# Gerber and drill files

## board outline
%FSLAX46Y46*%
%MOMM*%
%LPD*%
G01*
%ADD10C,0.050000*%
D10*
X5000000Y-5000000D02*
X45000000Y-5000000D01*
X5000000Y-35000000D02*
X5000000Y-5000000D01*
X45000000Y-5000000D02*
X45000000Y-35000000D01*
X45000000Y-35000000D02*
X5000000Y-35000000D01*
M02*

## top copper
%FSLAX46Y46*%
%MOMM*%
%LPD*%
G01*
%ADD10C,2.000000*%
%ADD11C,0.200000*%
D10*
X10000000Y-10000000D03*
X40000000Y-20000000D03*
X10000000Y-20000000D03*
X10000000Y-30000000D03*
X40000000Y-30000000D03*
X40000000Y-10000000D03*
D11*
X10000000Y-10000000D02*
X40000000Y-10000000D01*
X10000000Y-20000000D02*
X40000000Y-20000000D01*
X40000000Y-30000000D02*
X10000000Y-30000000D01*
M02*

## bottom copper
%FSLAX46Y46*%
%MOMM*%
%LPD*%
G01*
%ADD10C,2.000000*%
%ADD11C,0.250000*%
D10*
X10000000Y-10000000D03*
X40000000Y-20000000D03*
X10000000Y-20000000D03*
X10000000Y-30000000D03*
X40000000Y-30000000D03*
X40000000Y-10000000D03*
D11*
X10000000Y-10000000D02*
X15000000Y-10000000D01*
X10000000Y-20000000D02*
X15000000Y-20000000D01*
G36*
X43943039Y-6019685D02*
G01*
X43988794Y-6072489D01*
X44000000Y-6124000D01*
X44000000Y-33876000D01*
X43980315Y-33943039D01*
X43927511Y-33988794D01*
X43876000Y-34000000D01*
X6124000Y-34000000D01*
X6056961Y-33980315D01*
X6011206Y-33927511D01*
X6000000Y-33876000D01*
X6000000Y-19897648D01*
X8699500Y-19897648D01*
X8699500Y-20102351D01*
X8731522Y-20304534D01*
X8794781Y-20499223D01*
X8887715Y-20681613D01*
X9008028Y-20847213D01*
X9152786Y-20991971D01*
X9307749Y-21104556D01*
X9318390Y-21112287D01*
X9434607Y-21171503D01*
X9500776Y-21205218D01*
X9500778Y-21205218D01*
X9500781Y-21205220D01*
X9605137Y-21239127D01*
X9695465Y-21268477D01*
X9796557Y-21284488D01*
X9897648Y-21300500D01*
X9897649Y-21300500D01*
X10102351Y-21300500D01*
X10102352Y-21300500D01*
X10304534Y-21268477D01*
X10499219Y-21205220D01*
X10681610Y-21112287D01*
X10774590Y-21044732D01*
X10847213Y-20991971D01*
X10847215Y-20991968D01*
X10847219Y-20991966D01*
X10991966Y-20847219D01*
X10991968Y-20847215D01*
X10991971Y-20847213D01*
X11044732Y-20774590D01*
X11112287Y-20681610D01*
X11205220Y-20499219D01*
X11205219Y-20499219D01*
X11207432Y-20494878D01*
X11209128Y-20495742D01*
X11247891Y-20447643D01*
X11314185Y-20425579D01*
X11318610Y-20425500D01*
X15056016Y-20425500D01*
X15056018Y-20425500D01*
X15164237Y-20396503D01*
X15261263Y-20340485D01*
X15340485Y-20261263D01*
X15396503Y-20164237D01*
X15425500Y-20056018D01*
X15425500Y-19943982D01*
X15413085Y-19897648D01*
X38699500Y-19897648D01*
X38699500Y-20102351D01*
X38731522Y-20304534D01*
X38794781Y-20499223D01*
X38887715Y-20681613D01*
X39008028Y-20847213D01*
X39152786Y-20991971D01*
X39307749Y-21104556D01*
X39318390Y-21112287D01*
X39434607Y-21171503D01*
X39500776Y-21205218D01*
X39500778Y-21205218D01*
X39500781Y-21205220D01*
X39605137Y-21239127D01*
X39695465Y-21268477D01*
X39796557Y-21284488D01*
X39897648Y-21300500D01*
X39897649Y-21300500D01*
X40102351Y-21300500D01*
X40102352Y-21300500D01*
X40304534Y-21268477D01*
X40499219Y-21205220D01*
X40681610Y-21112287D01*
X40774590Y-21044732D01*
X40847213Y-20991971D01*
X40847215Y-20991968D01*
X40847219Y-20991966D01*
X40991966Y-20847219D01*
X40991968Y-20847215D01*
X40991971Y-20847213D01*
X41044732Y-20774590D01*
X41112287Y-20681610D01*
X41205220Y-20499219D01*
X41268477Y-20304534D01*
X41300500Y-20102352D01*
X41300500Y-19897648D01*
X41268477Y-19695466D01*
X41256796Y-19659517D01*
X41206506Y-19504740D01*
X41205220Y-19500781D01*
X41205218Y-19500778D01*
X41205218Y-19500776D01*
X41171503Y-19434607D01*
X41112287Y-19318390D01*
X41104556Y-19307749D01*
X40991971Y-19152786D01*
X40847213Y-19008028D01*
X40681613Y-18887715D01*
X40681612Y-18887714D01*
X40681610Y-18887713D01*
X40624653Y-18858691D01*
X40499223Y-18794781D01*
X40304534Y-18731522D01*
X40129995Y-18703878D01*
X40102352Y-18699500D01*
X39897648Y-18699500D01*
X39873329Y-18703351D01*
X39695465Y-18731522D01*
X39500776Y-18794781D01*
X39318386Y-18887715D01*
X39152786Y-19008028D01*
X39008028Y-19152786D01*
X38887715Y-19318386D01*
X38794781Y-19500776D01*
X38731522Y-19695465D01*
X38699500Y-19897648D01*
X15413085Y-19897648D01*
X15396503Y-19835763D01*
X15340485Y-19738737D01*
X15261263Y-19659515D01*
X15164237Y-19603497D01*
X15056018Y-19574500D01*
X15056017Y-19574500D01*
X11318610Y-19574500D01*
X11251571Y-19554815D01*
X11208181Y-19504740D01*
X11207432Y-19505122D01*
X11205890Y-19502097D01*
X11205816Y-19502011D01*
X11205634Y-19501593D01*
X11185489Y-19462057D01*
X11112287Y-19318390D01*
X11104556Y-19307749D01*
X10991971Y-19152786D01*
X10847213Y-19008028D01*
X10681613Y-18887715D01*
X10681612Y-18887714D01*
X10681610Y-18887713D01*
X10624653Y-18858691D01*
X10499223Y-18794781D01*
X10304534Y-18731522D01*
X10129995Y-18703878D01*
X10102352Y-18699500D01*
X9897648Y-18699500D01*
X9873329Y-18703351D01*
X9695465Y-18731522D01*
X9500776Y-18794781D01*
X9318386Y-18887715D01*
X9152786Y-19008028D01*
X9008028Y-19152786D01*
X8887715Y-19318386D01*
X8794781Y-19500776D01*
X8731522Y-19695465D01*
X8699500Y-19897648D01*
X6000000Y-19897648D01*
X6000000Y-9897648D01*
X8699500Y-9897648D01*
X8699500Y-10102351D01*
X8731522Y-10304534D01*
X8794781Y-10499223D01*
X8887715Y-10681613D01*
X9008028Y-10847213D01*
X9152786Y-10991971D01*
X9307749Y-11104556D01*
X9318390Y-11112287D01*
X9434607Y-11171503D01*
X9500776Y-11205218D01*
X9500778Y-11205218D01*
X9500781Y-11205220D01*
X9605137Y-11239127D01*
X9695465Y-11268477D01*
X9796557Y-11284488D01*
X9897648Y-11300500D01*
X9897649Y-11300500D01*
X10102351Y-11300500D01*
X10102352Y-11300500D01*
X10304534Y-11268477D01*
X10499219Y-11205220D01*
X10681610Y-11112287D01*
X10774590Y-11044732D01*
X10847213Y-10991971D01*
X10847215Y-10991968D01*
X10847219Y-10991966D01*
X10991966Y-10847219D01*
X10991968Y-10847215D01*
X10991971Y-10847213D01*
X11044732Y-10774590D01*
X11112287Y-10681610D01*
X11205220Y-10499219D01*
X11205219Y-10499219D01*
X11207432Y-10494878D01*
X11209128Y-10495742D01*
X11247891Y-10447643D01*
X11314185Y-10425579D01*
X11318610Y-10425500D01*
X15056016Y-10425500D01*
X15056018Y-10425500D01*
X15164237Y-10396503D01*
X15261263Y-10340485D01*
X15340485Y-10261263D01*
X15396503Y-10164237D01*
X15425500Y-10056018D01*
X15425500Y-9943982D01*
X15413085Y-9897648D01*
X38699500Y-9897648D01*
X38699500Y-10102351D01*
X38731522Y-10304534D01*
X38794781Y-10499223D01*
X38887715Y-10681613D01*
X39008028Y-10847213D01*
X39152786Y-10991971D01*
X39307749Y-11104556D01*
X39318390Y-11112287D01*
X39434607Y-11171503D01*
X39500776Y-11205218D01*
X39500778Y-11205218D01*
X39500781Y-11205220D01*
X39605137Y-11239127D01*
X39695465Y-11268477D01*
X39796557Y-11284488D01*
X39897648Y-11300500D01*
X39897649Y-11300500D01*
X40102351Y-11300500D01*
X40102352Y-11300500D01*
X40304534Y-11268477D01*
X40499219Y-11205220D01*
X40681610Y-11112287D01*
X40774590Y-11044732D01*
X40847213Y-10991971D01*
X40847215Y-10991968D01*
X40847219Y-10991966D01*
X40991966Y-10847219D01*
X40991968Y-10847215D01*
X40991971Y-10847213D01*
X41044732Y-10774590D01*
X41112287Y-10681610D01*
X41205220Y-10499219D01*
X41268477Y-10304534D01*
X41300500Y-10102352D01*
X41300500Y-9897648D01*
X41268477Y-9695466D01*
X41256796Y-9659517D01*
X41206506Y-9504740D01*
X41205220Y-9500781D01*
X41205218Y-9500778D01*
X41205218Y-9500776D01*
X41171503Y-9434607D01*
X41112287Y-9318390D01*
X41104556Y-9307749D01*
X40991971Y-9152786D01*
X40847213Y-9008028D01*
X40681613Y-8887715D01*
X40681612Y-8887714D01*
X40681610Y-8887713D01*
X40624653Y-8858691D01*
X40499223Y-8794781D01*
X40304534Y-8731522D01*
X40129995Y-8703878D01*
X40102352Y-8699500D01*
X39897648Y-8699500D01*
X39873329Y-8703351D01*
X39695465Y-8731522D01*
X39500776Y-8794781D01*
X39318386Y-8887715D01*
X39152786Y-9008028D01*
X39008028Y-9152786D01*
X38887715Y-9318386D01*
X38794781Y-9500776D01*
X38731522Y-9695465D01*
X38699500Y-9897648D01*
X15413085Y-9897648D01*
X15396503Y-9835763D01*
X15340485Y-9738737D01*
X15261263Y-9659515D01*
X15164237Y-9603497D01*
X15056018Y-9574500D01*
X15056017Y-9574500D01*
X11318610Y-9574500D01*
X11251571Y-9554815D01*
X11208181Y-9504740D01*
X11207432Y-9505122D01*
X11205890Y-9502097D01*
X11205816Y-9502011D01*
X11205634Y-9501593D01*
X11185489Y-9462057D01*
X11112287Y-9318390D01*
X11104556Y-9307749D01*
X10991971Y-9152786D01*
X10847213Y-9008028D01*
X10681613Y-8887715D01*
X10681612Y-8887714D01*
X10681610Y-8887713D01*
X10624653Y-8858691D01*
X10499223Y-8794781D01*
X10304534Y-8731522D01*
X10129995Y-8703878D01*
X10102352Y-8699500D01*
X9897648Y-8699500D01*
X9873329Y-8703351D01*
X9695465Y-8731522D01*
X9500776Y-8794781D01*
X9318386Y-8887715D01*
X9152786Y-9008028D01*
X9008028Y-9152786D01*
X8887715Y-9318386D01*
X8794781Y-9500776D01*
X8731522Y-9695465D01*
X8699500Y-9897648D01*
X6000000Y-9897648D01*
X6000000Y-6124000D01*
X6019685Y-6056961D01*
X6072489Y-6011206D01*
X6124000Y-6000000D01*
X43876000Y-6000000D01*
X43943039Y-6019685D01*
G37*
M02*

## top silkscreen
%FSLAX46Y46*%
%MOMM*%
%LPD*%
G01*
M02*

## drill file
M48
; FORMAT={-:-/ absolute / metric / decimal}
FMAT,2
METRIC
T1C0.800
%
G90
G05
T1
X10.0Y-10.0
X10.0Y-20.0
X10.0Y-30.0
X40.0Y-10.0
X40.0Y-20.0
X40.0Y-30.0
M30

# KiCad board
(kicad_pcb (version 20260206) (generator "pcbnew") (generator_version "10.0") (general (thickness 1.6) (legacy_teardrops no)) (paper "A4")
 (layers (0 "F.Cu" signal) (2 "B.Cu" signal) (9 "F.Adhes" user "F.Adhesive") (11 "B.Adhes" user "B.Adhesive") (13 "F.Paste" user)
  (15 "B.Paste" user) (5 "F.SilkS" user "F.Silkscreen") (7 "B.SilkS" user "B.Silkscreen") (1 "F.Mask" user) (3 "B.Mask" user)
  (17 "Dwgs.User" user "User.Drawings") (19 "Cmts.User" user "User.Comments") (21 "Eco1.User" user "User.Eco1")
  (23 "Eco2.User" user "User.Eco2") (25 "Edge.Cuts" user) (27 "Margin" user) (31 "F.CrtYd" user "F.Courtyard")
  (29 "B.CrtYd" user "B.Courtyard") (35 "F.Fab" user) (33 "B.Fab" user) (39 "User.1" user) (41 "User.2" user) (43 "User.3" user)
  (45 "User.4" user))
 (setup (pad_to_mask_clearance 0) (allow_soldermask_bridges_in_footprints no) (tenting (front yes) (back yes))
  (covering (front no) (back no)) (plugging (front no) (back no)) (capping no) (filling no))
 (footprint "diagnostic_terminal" (layer "F.Cu") (at 10 10)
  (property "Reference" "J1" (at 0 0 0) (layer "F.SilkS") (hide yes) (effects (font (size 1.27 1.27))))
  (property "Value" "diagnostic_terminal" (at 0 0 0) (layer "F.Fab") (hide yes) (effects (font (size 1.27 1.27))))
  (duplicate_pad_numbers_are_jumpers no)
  (pad "1" thru_hole circle (at 0 0) (size 2 2) (drill 0.8) (layers "*.Cu") (remove_unused_layers no) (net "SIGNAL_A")))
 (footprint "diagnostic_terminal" (layer "F.Cu") (at 40 20)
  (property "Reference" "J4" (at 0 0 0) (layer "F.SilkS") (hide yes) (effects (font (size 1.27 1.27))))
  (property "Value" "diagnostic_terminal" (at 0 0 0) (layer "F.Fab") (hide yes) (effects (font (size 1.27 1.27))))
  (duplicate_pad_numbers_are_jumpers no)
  (pad "1" thru_hole circle (at 0 0) (size 2 2) (drill 0.8) (layers "*.Cu") (remove_unused_layers no) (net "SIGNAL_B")))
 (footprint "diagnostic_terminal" (layer "F.Cu") (at 10 20)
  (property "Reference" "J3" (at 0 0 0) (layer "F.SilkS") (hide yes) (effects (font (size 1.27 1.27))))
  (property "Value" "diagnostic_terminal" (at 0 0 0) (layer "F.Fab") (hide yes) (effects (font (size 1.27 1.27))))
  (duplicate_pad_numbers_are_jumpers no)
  (pad "1" thru_hole circle (at 0 0) (size 2 2) (drill 0.8) (layers "*.Cu") (remove_unused_layers no) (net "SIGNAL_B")))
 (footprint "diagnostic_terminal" (layer "F.Cu") (at 10 30)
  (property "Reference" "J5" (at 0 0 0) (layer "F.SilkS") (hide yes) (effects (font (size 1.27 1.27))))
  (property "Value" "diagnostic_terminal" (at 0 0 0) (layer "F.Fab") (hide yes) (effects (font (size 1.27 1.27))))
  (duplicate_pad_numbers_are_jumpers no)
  (pad "1" thru_hole circle (at 0 0) (size 2 2) (drill 0.8) (layers "*.Cu") (remove_unused_layers no) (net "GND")))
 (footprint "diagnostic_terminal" (layer "F.Cu") (at 40 30)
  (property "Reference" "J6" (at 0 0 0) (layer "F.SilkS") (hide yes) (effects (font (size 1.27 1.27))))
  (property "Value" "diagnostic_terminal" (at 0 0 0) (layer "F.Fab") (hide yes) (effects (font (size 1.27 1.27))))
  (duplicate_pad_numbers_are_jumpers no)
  (pad "1" thru_hole circle (at 0 0) (size 2 2) (drill 0.8) (layers "*.Cu") (remove_unused_layers no) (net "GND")))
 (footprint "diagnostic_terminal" (layer "F.Cu") (at 40 10)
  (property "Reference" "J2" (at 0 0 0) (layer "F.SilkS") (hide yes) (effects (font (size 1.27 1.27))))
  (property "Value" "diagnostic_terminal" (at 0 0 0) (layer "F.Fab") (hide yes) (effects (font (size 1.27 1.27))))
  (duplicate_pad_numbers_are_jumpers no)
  (pad "1" thru_hole circle (at 0 0) (size 2 2) (drill 0.8) (layers "*.Cu") (remove_unused_layers no) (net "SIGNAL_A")))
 (gr_line (start 5 5) (end 45 5) (stroke (width 0.05) (type default)) (layer "Edge.Cuts"))
 (gr_line (start 5 35) (end 5 5) (stroke (width 0.05) (type default)) (layer "Edge.Cuts"))
 (gr_line (start 45 5) (end 45 35) (stroke (width 0.05) (type default)) (layer "Edge.Cuts"))
 (gr_line (start 45 35) (end 5 35) (stroke (width 0.05) (type default)) (layer "Edge.Cuts"))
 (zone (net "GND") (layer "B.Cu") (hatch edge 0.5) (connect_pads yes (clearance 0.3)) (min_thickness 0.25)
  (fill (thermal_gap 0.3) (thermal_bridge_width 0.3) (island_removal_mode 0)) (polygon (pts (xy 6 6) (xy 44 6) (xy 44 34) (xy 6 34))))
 (segment (start 10 10) (end 40 10) (width 0.2) (layer "F.Cu") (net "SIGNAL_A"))
 (segment (start 10 10) (end 15 10) (width 0.25) (layer "B.Cu") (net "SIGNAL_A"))
 (segment (start 10 20) (end 40 20) (width 0.2) (layer "F.Cu") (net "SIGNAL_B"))
 (segment (start 10 20) (end 15 20) (width 0.25) (layer "B.Cu") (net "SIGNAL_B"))
 (segment (start 40 30) (end 10 30) (width 0.2) (layer "F.Cu") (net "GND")))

